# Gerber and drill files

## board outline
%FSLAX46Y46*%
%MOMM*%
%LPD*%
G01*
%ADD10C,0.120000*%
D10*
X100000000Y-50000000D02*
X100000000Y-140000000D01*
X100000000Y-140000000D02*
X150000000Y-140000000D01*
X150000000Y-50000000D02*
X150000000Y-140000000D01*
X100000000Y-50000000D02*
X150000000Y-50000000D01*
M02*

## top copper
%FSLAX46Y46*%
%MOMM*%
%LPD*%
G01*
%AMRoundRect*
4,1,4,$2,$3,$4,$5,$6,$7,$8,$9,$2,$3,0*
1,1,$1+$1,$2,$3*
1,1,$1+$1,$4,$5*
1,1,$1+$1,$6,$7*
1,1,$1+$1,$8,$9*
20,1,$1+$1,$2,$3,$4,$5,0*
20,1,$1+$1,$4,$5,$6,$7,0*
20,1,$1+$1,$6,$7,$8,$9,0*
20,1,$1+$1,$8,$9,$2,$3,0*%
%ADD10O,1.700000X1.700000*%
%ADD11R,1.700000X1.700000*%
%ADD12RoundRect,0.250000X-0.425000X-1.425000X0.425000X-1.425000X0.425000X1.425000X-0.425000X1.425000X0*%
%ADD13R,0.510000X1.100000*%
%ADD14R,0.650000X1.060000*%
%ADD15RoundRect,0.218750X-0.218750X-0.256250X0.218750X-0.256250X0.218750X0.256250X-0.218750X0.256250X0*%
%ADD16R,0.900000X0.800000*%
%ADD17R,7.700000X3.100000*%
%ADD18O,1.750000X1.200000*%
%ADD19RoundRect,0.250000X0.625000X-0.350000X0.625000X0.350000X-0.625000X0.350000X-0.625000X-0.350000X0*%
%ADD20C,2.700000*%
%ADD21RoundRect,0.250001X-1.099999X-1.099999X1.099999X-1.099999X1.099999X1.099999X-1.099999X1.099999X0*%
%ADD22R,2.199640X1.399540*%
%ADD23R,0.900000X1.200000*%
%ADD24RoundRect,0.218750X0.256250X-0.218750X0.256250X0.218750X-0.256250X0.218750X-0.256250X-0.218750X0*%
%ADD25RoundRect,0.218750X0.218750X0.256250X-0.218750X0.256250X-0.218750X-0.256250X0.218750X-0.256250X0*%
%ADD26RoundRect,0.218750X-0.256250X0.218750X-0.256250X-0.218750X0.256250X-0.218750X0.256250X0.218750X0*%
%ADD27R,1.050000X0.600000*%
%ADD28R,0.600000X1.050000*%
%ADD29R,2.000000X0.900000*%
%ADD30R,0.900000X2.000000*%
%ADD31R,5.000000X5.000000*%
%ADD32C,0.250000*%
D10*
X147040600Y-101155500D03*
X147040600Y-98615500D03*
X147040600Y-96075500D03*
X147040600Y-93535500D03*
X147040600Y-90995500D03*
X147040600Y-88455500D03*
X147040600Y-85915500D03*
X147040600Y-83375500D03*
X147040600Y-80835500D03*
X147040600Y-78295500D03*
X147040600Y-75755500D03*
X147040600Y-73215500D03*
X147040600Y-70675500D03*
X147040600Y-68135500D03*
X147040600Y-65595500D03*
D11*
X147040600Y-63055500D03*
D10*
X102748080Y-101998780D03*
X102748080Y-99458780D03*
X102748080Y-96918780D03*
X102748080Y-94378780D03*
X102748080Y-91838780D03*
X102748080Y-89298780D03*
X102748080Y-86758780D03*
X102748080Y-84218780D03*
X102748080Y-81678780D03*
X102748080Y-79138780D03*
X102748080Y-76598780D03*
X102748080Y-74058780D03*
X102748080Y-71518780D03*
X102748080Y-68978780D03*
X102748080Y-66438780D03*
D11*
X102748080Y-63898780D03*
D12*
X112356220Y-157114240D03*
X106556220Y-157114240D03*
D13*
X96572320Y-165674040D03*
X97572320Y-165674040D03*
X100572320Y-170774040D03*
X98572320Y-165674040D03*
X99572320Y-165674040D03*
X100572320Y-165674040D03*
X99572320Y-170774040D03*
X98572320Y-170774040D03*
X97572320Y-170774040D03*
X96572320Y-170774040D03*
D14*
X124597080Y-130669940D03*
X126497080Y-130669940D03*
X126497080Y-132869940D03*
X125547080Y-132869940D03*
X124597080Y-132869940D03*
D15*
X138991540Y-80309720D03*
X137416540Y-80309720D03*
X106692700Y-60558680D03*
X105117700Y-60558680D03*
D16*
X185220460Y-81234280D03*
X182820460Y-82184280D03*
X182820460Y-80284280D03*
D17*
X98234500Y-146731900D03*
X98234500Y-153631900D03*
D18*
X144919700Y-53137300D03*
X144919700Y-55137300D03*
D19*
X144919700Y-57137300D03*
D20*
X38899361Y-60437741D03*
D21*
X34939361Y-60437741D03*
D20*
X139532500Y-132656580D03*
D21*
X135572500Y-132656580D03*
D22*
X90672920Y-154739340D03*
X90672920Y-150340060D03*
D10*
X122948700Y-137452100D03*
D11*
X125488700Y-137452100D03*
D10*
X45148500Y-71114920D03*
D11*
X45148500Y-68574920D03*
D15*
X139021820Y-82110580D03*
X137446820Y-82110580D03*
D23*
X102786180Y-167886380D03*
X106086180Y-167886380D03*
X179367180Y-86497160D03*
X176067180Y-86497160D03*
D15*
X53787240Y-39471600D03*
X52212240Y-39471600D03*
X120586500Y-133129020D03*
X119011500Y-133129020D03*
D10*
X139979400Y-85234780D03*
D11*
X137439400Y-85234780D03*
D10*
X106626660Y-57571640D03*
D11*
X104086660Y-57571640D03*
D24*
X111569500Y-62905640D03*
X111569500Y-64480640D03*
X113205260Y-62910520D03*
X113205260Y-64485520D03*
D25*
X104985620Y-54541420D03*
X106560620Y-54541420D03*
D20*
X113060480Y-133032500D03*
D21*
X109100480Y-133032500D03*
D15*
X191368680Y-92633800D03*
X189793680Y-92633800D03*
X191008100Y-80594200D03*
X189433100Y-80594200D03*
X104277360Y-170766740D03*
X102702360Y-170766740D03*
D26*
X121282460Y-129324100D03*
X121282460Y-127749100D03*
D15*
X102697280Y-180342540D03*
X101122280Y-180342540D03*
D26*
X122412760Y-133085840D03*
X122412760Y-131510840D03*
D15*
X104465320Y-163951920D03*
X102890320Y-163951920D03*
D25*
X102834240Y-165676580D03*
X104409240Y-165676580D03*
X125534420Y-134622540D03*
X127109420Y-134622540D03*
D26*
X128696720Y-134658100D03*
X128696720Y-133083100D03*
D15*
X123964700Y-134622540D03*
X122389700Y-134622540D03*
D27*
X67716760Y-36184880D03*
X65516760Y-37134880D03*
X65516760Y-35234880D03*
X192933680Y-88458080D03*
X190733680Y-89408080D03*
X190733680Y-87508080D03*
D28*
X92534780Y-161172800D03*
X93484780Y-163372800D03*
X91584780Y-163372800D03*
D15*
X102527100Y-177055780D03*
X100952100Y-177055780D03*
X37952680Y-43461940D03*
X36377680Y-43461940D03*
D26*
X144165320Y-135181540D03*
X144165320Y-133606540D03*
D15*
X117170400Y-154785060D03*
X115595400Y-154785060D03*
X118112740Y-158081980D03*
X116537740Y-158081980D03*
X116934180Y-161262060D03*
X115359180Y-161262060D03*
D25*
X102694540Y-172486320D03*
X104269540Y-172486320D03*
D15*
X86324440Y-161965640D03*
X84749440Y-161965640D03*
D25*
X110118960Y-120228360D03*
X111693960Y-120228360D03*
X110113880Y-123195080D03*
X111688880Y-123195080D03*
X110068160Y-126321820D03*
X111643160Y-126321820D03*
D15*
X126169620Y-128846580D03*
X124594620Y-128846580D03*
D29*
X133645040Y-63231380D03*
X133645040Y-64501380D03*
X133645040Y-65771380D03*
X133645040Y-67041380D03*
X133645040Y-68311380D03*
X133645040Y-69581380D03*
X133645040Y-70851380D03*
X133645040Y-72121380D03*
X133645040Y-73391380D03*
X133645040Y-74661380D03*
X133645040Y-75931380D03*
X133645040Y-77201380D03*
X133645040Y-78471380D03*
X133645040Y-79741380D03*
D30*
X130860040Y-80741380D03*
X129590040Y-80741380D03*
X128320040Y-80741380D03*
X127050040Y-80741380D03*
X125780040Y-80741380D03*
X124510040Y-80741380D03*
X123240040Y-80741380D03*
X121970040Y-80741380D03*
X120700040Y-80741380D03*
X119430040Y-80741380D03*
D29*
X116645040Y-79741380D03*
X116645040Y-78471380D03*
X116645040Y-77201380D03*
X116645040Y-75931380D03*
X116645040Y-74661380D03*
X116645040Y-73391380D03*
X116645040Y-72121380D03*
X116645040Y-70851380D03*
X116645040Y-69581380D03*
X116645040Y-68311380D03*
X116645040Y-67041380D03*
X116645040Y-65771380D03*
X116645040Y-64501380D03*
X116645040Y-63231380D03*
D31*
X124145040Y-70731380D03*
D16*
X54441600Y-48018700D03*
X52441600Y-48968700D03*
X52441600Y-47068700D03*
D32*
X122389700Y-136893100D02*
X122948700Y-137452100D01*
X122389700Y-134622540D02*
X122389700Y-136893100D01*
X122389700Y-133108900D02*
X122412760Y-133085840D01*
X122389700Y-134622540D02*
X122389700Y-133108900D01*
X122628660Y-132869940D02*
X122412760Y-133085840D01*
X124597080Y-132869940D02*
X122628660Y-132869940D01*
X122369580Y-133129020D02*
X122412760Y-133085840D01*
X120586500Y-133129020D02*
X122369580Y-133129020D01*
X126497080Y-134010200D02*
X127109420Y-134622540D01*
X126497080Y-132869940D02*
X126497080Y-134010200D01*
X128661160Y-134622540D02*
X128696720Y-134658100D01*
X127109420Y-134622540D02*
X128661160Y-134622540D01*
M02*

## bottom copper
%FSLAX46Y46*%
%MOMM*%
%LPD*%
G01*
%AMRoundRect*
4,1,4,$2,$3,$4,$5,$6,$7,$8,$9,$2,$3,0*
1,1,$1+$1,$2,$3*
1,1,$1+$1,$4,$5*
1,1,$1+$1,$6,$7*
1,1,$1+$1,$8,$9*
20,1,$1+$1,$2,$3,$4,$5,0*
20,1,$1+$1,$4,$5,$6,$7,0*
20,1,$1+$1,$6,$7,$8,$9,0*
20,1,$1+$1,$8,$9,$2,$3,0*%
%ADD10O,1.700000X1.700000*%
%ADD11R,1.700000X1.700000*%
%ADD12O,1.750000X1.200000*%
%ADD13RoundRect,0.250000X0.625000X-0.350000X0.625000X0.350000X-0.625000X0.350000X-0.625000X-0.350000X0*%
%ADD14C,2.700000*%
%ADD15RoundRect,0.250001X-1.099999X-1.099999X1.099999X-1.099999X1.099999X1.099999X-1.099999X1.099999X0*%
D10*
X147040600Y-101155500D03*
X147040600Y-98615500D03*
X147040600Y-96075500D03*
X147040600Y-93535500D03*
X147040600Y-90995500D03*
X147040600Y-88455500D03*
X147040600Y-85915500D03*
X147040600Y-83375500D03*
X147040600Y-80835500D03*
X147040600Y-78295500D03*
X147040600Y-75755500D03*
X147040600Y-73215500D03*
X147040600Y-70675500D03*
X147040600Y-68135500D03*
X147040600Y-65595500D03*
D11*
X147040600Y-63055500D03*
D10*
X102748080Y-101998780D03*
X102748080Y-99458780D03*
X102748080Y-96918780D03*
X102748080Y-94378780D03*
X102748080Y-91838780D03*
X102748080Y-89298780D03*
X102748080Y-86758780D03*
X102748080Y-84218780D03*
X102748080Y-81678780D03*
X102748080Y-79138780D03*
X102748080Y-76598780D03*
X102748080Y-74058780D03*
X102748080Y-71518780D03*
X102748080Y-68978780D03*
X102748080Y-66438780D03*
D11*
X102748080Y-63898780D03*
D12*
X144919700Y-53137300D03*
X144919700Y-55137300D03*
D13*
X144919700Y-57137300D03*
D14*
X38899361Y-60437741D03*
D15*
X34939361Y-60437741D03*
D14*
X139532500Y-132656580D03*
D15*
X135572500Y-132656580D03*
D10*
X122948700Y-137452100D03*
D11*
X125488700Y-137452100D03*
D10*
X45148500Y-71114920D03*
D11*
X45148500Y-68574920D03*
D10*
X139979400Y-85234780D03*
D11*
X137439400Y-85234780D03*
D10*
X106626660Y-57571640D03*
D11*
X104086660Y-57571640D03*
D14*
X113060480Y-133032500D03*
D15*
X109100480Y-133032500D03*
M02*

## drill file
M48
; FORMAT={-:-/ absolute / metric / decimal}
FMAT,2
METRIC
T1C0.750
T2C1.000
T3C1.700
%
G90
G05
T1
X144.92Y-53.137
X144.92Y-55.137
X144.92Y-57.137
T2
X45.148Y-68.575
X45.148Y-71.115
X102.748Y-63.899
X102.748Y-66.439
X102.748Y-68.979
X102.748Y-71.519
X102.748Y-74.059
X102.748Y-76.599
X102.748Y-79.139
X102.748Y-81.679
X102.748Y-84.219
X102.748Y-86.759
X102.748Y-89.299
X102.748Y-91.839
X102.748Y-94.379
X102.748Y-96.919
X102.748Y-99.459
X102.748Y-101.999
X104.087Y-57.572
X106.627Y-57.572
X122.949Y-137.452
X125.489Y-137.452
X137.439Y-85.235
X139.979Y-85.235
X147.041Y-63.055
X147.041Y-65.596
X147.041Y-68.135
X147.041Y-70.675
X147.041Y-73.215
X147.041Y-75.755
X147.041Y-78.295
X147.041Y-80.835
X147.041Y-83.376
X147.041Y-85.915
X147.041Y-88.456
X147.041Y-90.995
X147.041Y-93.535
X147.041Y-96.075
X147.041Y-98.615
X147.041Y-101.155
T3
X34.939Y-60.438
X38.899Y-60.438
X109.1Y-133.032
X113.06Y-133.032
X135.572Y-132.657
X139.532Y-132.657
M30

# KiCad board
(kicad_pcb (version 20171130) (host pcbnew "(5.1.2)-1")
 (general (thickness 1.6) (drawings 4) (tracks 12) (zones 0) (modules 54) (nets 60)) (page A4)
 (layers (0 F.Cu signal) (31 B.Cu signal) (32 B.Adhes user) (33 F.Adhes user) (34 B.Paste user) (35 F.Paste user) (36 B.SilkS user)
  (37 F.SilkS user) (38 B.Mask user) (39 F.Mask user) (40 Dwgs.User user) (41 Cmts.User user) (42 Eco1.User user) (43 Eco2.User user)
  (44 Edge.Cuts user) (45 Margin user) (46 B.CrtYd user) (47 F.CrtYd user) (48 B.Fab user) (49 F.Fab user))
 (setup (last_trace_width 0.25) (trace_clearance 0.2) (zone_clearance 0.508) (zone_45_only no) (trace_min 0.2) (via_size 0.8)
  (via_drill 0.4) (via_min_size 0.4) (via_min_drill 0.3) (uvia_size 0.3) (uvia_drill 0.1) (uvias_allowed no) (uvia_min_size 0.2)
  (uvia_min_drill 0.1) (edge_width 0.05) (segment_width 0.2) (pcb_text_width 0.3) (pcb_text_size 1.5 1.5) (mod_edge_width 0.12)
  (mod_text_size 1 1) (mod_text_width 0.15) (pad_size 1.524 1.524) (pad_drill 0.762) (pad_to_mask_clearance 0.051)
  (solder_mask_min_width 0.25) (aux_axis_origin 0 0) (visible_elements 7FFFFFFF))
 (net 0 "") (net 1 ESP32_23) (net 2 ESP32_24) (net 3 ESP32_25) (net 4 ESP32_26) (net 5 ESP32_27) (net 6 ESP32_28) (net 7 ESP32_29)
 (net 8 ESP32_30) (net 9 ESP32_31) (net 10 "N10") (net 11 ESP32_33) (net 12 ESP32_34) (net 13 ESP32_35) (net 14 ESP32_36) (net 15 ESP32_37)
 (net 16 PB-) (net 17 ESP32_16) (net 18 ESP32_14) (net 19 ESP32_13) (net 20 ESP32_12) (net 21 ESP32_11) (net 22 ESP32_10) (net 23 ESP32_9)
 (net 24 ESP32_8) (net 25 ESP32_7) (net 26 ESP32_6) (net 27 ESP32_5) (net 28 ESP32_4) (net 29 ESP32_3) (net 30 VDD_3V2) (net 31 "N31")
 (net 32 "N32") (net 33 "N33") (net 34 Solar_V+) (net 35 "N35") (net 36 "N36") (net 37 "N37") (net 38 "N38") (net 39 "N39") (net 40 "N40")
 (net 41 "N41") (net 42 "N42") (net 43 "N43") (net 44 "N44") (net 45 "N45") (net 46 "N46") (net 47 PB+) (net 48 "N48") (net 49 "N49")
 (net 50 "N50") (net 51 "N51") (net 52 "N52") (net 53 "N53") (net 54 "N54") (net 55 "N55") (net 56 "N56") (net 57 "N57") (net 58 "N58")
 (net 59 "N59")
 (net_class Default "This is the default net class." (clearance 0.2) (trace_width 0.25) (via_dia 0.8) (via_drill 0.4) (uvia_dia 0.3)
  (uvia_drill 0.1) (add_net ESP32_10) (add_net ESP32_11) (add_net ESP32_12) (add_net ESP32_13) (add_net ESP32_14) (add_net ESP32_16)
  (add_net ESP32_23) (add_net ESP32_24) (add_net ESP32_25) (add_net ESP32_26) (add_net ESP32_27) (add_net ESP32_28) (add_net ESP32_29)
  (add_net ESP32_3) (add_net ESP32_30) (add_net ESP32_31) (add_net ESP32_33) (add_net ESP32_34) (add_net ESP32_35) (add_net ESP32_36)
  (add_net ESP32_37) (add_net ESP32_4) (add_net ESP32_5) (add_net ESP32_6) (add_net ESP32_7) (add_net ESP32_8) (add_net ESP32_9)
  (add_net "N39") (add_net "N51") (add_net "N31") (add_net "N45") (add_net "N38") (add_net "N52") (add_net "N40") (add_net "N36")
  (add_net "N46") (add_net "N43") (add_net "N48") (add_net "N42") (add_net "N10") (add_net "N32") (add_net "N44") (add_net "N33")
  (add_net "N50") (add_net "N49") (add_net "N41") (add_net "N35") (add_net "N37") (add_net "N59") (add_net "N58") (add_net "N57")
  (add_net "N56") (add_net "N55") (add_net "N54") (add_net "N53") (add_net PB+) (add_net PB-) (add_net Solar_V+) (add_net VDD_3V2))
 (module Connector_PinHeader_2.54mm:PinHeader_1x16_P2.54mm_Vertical (layer F.Cu) (at 147.0406 63.0555)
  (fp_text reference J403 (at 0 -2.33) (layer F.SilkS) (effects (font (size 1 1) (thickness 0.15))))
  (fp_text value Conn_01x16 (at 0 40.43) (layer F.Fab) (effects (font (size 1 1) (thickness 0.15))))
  (pad 16 thru_hole oval (at 0 38.1) (size 1.7 1.7) (drill 1) (layers *.Cu *.Mask) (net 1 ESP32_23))
  (pad 15 thru_hole oval (at 0 35.56) (size 1.7 1.7) (drill 1) (layers *.Cu *.Mask) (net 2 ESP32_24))
  (pad 14 thru_hole oval (at 0 33.02) (size 1.7 1.7) (drill 1) (layers *.Cu *.Mask) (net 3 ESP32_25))
  (pad 13 thru_hole oval (at 0 30.48) (size 1.7 1.7) (drill 1) (layers *.Cu *.Mask) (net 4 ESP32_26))
  (pad 12 thru_hole oval (at 0 27.94) (size 1.7 1.7) (drill 1) (layers *.Cu *.Mask) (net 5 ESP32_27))
  (pad 11 thru_hole oval (at 0 25.4) (size 1.7 1.7) (drill 1) (layers *.Cu *.Mask) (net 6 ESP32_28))
  (pad 10 thru_hole oval (at 0 22.86) (size 1.7 1.7) (drill 1) (layers *.Cu *.Mask) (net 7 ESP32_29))
  (pad 9 thru_hole oval (at 0 20.32) (size 1.7 1.7) (drill 1) (layers *.Cu *.Mask) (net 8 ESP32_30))
  (pad 8 thru_hole oval (at 0 17.78) (size 1.7 1.7) (drill 1) (layers *.Cu *.Mask) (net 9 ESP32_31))
  (pad 7 thru_hole oval (at 0 15.24) (size 1.7 1.7) (drill 1) (layers *.Cu *.Mask) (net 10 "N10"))
  (pad 6 thru_hole oval (at 0 12.7) (size 1.7 1.7) (drill 1) (layers *.Cu *.Mask) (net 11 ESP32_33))
  (pad 5 thru_hole oval (at 0 10.16) (size 1.7 1.7) (drill 1) (layers *.Cu *.Mask) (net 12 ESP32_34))
  (pad 4 thru_hole oval (at 0 7.62) (size 1.7 1.7) (drill 1) (layers *.Cu *.Mask) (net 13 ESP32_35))
  (pad 3 thru_hole oval (at 0 5.08) (size 1.7 1.7) (drill 1) (layers *.Cu *.Mask) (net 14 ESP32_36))
  (pad 2 thru_hole oval (at 0 2.54) (size 1.7 1.7) (drill 1) (layers *.Cu *.Mask) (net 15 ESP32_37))
  (pad 1 thru_hole rect (at 0 0) (size 1.7 1.7) (drill 1) (layers *.Cu *.Mask) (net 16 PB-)))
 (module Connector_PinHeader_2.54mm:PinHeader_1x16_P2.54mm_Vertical (layer F.Cu) (at 102.74808 63.89878)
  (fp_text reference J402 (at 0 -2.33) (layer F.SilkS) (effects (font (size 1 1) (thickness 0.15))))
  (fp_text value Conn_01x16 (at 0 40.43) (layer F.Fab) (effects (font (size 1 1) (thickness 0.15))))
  (pad 16 thru_hole oval (at 0 38.1) (size 1.7 1.7) (drill 1) (layers *.Cu *.Mask) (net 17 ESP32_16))
  (pad 15 thru_hole oval (at 0 35.56) (size 1.7 1.7) (drill 1) (layers *.Cu *.Mask) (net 16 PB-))
  (pad 14 thru_hole oval (at 0 33.02) (size 1.7 1.7) (drill 1) (layers *.Cu *.Mask) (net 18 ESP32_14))
  (pad 13 thru_hole oval (at 0 30.48) (size 1.7 1.7) (drill 1) (layers *.Cu *.Mask) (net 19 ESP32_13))
  (pad 12 thru_hole oval (at 0 27.94) (size 1.7 1.7) (drill 1) (layers *.Cu *.Mask) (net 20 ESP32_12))
  (pad 11 thru_hole oval (at 0 25.4) (size 1.7 1.7) (drill 1) (layers *.Cu *.Mask) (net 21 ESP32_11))
  (pad 10 thru_hole oval (at 0 22.86) (size 1.7 1.7) (drill 1) (layers *.Cu *.Mask) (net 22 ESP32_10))
  (pad 9 thru_hole oval (at 0 20.32) (size 1.7 1.7) (drill 1) (layers *.Cu *.Mask) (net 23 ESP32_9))
  (pad 8 thru_hole oval (at 0 17.78) (size 1.7 1.7) (drill 1) (layers *.Cu *.Mask) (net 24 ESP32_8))
  (pad 7 thru_hole oval (at 0 15.24) (size 1.7 1.7) (drill 1) (layers *.Cu *.Mask) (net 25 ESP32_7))
  (pad 6 thru_hole oval (at 0 12.7) (size 1.7 1.7) (drill 1) (layers *.Cu *.Mask) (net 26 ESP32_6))
  (pad 5 thru_hole oval (at 0 10.16) (size 1.7 1.7) (drill 1) (layers *.Cu *.Mask) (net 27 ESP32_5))
  (pad 4 thru_hole oval (at 0 7.62) (size 1.7 1.7) (drill 1) (layers *.Cu *.Mask) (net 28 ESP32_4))
  (pad 3 thru_hole oval (at 0 5.08) (size 1.7 1.7) (drill 1) (layers *.Cu *.Mask) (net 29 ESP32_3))
  (pad 2 thru_hole oval (at 0 2.54) (size 1.7 1.7) (drill 1) (layers *.Cu *.Mask) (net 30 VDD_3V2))
  (pad 1 thru_hole rect (at 0 0) (size 1.7 1.7) (drill 1) (layers *.Cu *.Mask) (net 16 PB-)))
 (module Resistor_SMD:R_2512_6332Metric (layer F.Cu) (at 109.45622 157.11424)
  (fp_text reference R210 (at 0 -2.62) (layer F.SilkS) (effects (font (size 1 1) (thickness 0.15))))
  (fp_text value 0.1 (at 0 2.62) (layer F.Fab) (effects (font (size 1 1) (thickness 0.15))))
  (pad 2 smd roundrect (at 2.9 0) (size 1.35 3.35) (layers F.Cu F.Paste F.Mask) (roundrect_rratio 0.185185) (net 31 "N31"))
  (pad 1 smd roundrect (at -2.9 0) (size 1.35 3.35) (layers F.Cu F.Paste F.Mask) (roundrect_rratio 0.185185) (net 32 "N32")))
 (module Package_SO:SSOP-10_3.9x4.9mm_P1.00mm (layer F.Cu) (at 98.57232 168.22404 90)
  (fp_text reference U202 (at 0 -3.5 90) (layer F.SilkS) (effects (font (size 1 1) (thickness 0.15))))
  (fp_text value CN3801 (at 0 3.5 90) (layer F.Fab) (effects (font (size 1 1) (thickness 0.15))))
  (pad 10 smd rect (at 2.55 -2 90) (size 1.1 0.51) (layers F.Cu F.Paste F.Mask) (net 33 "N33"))
  (pad 9 smd rect (at 2.55 -1 90) (size 1.1 0.51) (layers F.Cu F.Paste F.Mask) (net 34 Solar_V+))
  (pad 5 smd rect (at -2.55 2 90) (size 1.1 0.51) (layers F.Cu F.Paste F.Mask) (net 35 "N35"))
  (pad 8 smd rect (at 2.55 0 90) (size 1.1 0.51) (layers F.Cu F.Paste F.Mask) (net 32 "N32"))
  (pad 7 smd rect (at 2.55 1 90) (size 1.1 0.51) (layers F.Cu F.Paste F.Mask) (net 31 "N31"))
  (pad 6 smd rect (at 2.55 2 90) (size 1.1 0.51) (layers F.Cu F.Paste F.Mask) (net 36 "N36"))
  (pad 4 smd rect (at -2.55 1 90) (size 1.1 0.51) (layers F.Cu F.Paste F.Mask) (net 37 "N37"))
  (pad 3 smd rect (at -2.55 0 90) (size 1.1 0.51) (layers F.Cu F.Paste F.Mask) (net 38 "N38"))
  (pad 2 smd rect (at -2.55 -1 90) (size 1.1 0.51) (layers F.Cu F.Paste F.Mask) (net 16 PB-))
  (pad 1 smd rect (at -2.55 -2 90) (size 1.1 0.51) (layers F.Cu F.Paste F.Mask) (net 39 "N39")))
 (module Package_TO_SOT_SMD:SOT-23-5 (layer F.Cu) (at 125.54708 131.76994 90)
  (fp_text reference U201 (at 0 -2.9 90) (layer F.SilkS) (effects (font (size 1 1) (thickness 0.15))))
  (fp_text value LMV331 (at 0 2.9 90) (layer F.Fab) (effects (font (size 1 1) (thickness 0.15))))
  (pad 5 smd rect (at 1.1 -0.95 90) (size 1.06 0.65) (layers F.Cu F.Paste F.Mask) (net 34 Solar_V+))
  (pad 4 smd rect (at 1.1 0.95 90) (size 1.06 0.65) (layers F.Cu F.Paste F.Mask) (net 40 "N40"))
  (pad 3 smd rect (at -1.1 0.95 90) (size 1.06 0.65) (layers F.Cu F.Paste F.Mask) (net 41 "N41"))
  (pad 2 smd rect (at -1.1 0 90) (size 1.06 0.65) (layers F.Cu F.Paste F.Mask) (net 16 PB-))
  (pad 1 smd rect (at -1.1 -0.95 90) (size 1.06 0.65) (layers F.Cu F.Paste F.Mask) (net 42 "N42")))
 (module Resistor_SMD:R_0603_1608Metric (layer F.Cu) (at 138.20404 80.30972)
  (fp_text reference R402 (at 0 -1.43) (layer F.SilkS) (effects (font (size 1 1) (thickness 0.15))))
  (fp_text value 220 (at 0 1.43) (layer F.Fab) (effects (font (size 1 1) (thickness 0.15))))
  (pad 2 smd roundrect (at 0.7875 0) (size 0.875 0.95) (layers F.Cu F.Paste F.Mask) (roundrect_rratio 0.25) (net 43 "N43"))
  (pad 1 smd roundrect (at -0.7875 0) (size 0.875 0.95) (layers F.Cu F.Paste F.Mask) (roundrect_rratio 0.25) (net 30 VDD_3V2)))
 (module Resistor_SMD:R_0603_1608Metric (layer F.Cu) (at 105.9052 60.55868)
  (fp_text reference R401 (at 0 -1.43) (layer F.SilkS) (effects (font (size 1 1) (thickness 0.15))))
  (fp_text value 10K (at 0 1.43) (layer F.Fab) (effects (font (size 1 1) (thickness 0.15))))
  (pad 2 smd roundrect (at 0.7875 0) (size 0.875 0.95) (layers F.Cu F.Paste F.Mask) (roundrect_rratio 0.25) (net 29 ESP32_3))
  (pad 1 smd roundrect (at -0.7875 0) (size 0.875 0.95) (layers F.Cu F.Paste F.Mask) (roundrect_rratio 0.25) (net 30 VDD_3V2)))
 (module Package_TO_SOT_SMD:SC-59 (layer F.Cu) (at 184.02046 81.23428)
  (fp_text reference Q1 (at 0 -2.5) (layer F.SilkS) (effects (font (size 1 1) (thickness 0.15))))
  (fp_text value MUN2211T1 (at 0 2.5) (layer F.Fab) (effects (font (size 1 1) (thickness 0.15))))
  (pad 3 smd rect (at 1.2 0) (size 0.9 0.8) (layers F.Cu F.Paste F.Mask) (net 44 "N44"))
  (pad 2 smd rect (at -1.2 0.95) (size 0.9 0.8) (layers F.Cu F.Paste F.Mask) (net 16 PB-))
  (pad 1 smd rect (at -1.2 -0.95) (size 0.9 0.8) (layers F.Cu F.Paste F.Mask) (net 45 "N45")))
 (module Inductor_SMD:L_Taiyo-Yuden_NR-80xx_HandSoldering (layer F.Cu) (at 98.2345 150.1819 90)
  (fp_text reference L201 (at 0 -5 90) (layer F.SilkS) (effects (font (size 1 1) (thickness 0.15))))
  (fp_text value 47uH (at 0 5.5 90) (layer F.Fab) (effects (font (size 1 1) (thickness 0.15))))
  (pad 2 smd rect (at 3.45 0 90) (size 3.1 7.7) (layers F.Cu F.Paste F.Mask) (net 32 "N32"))
  (pad 1 smd rect (at -3.45 0 90) (size 3.1 7.7) (layers F.Cu F.Paste F.Mask) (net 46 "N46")))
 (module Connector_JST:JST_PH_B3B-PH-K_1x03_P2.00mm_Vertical (layer F.Cu) (at 144.9197 57.1373 90)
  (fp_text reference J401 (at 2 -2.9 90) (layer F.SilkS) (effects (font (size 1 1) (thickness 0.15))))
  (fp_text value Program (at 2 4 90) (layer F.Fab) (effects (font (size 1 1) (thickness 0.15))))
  (pad 3 thru_hole oval (at 4 0 90) (size 1.2 1.75) (drill 0.75) (layers *.Cu *.Mask) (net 13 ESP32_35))
  (pad 2 thru_hole oval (at 2 0 90) (size 1.2 1.75) (drill 0.75) (layers *.Cu *.Mask) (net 12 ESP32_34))
  (pad 1 thru_hole roundrect (at 0 0 90) (size 1.2 1.75) (drill 0.75) (layers *.Cu *.Mask) (roundrect_rratio 0.208333) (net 16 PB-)))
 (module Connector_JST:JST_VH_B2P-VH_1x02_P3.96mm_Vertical (layer F.Cu) (at 34.939361 60.437741)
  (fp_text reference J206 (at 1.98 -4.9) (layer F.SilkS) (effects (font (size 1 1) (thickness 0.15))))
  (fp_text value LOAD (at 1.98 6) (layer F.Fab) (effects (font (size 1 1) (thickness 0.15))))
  (pad 2 thru_hole circle (at 3.96 0) (size 2.7 2.7) (drill 1.7) (layers *.Cu *.Mask) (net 30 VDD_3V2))
  (pad 1 thru_hole roundrect (at 0 0) (size 2.7 2.7) (drill 1.7) (layers *.Cu *.Mask) (roundrect_rratio 0.09259299999999999) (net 16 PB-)))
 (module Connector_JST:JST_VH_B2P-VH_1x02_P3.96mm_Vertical (layer F.Cu) (at 135.5725 132.65658)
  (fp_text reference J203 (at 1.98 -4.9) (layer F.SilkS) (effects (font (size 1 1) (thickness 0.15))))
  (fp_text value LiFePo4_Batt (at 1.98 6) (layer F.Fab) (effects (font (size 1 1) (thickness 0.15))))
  (pad 2 thru_hole circle (at 3.96 0) (size 2.7 2.7) (drill 1.7) (layers *.Cu *.Mask) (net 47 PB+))
  (pad 1 thru_hole roundrect (at 0 0) (size 2.7 2.7) (drill 1.7) (layers *.Cu *.Mask) (roundrect_rratio 0.09259299999999999) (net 16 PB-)))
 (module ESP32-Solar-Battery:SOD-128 (layer F.Cu) (at 90.67292 152.5397 270)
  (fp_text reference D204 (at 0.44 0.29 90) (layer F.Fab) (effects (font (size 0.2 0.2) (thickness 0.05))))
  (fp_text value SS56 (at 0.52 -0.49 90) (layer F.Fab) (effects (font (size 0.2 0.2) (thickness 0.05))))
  (pad 1 smd rect (at 2.19964 0 270) (size 1.39954 2.19964) (layers F.Cu F.Paste F.Mask) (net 46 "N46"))
  (pad 2 smd rect (at -2.19964 0 270) (size 1.39954 2.19964) (layers F.Cu F.Paste F.Mask) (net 16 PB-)))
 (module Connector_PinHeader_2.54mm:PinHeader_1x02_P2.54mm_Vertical (layer F.Cu) (at 125.4887 137.4521 270)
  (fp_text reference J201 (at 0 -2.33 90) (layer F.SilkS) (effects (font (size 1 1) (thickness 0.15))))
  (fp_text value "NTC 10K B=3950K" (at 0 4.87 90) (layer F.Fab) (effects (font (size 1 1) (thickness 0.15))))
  (pad 2 thru_hole oval (at 0 2.54 270) (size 1.7 1.7) (drill 1) (layers *.Cu *.Mask) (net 42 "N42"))
  (pad 1 thru_hole rect (at 0 0 270) (size 1.7 1.7) (drill 1) (layers *.Cu *.Mask) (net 16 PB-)))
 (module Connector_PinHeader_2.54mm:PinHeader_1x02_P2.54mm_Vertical (layer F.Cu) (at 45.1485 68.57492)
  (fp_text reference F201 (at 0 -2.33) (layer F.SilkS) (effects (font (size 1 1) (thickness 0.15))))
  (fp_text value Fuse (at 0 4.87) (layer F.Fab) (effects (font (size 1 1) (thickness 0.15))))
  (pad 2 thru_hole oval (at 0 2.54) (size 1.7 1.7) (drill 1) (layers *.Cu *.Mask) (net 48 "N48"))
  (pad 1 thru_hole rect (at 0 0) (size 1.7 1.7) (drill 1) (layers *.Cu *.Mask) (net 30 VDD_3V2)))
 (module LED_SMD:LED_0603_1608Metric (layer F.Cu) (at 138.23432 82.11058)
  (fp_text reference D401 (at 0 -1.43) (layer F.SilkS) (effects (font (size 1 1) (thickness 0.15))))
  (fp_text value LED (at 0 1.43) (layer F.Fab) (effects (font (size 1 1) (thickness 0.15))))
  (pad 2 smd roundrect (at 0.7875 0) (size 0.875 0.95) (layers F.Cu F.Paste F.Mask) (roundrect_rratio 0.25) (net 43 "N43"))
  (pad 1 smd roundrect (at -0.7875 0) (size 0.875 0.95) (layers F.Cu F.Paste F.Mask) (roundrect_rratio 0.25) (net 3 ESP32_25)))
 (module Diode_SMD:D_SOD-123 (layer F.Cu) (at 104.43618 167.88638 180)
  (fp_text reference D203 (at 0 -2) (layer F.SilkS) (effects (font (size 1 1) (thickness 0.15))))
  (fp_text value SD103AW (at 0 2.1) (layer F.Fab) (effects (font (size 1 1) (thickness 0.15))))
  (pad 2 smd rect (at 1.65 0 180) (size 0.9 1.2) (layers F.Cu F.Paste F.Mask) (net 36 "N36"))
  (pad 1 smd rect (at -1.65 0 180) (size 0.9 1.2) (layers F.Cu F.Paste F.Mask) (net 40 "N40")))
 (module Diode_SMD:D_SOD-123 (layer F.Cu) (at 177.71718 86.49716)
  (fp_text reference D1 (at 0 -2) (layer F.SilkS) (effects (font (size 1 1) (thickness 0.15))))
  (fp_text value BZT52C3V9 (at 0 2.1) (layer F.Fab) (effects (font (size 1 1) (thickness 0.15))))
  (pad 2 smd rect (at 1.65 0) (size 0.9 1.2) (layers F.Cu F.Paste F.Mask) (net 45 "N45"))
  (pad 1 smd rect (at -1.65 0) (size 0.9 1.2) (layers F.Cu F.Paste F.Mask) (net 34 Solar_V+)))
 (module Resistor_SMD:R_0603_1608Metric (layer F.Cu) (at 52.99974 39.4716)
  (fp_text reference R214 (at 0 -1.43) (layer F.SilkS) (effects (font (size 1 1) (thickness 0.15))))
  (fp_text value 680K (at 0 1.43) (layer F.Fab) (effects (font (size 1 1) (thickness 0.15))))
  (pad 2 smd roundrect (at 0.7875 0) (size 0.875 0.95) (layers F.Cu F.Paste F.Mask) (roundrect_rratio 0.25) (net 47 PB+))
  (pad 1 smd roundrect (at -0.7875 0) (size 0.875 0.95) (layers F.Cu F.Paste F.Mask) (roundrect_rratio 0.25) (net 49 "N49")))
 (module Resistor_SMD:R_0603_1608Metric (layer F.Cu) (at 119.799 133.12902)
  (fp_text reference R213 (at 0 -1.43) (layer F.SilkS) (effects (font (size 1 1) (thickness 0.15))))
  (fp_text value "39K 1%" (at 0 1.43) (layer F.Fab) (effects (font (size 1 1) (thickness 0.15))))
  (pad 2 smd roundrect (at 0.7875 0) (size 0.875 0.95) (layers F.Cu F.Paste F.Mask) (roundrect_rratio 0.25) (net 42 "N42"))
  (pad 1 smd roundrect (at -0.7875 0) (size 0.875 0.95) (layers F.Cu F.Paste F.Mask) (roundrect_rratio 0.25) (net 34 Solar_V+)))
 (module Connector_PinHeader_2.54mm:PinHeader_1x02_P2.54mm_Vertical (layer F.Cu) (at 137.4394 85.23478 90)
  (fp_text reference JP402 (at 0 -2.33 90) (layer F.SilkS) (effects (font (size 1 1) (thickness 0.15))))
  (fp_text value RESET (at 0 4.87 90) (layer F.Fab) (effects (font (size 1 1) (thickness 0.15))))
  (pad 2 thru_hole oval (at 0 2.54 90) (size 1.7 1.7) (drill 1) (layers *.Cu *.Mask) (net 16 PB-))
  (pad 1 thru_hole rect (at 0 0 90) (size 1.7 1.7) (drill 1) (layers *.Cu *.Mask) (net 3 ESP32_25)))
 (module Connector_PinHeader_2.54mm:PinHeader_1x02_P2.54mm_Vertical (layer F.Cu) (at 104.08666 57.57164 90)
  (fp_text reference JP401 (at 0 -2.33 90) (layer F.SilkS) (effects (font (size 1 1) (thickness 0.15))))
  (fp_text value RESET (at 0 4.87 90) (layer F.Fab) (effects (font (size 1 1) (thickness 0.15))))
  (pad 2 thru_hole oval (at 0 2.54 90) (size 1.7 1.7) (drill 1) (layers *.Cu *.Mask) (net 29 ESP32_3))
  (pad 1 thru_hole rect (at 0 0 90) (size 1.7 1.7) (drill 1) (layers *.Cu *.Mask) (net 16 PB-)))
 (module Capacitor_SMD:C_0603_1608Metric (layer F.Cu) (at 111.5695 63.69314 90)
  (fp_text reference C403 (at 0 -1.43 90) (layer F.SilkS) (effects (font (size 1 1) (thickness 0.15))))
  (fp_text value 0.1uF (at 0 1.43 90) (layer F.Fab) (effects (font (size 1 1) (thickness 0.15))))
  (pad 2 smd roundrect (at 0.7875 0 90) (size 0.875 0.95) (layers F.Cu F.Paste F.Mask) (roundrect_rratio 0.25) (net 16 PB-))
  (pad 1 smd roundrect (at -0.7875 0 90) (size 0.875 0.95) (layers F.Cu F.Paste F.Mask) (roundrect_rratio 0.25) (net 30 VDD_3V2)))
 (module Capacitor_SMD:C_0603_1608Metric (layer F.Cu) (at 113.20526 63.69802 90)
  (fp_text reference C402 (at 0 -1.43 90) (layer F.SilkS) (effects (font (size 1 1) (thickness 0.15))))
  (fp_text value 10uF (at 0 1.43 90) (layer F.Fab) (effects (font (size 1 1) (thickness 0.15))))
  (pad 2 smd roundrect (at 0.7875 0 90) (size 0.875 0.95) (layers F.Cu F.Paste F.Mask) (roundrect_rratio 0.25) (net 16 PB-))
  (pad 1 smd roundrect (at -0.7875 0 90) (size 0.875 0.95) (layers F.Cu F.Paste F.Mask) (roundrect_rratio 0.25) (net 30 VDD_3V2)))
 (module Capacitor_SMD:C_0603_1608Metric (layer F.Cu) (at 105.77312 54.54142 180)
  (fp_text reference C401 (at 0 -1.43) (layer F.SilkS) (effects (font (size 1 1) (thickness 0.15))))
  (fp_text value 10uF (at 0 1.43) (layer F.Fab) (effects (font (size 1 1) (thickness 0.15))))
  (pad 2 smd roundrect (at 0.7875 0 180) (size 0.875 0.95) (layers F.Cu F.Paste F.Mask) (roundrect_rratio 0.25) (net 16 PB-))
  (pad 1 smd roundrect (at -0.7875 0 180) (size 0.875 0.95) (layers F.Cu F.Paste F.Mask) (roundrect_rratio 0.25) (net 29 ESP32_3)))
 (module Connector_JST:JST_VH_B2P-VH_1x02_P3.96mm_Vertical (layer F.Cu) (at 109.10048 133.0325)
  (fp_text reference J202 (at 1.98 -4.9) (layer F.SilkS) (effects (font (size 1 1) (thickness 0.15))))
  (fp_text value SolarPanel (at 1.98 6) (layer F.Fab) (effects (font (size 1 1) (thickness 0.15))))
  (pad 2 thru_hole circle (at 3.96 0) (size 2.7 2.7) (drill 1.7) (layers *.Cu *.Mask) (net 34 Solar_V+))
  (pad 1 thru_hole roundrect (at 0 0) (size 2.7 2.7) (drill 1.7) (layers *.Cu *.Mask) (roundrect_rratio 0.09259299999999999) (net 16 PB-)))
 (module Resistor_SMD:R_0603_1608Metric (layer F.Cu) (at 190.58118 92.6338)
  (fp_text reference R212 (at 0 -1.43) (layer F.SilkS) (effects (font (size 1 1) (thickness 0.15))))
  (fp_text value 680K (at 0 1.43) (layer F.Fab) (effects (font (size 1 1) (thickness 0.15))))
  (pad 2 smd roundrect (at 0.7875 0) (size 0.875 0.95) (layers F.Cu F.Paste F.Mask) (roundrect_rratio 0.25) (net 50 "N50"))
  (pad 1 smd roundrect (at -0.7875 0) (size 0.875 0.95) (layers F.Cu F.Paste F.Mask) (roundrect_rratio 0.25) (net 47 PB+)))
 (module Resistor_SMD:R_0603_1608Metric (layer F.Cu) (at 190.2206 80.5942)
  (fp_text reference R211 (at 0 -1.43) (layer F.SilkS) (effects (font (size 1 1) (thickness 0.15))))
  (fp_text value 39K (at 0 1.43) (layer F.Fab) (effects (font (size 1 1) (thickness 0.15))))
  (pad 2 smd roundrect (at 0.7875 0) (size 0.875 0.95) (layers F.Cu F.Paste F.Mask) (roundrect_rratio 0.25) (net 44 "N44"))
  (pad 1 smd roundrect (at -0.7875 0) (size 0.875 0.95) (layers F.Cu F.Paste F.Mask) (roundrect_rratio 0.25) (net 50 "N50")))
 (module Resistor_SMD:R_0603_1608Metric (layer F.Cu) (at 103.48986 170.76674)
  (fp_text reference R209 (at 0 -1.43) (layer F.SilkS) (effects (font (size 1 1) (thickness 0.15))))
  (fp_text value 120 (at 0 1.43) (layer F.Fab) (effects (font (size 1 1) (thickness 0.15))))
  (pad 2 smd roundrect (at 0.7875 0) (size 0.875 0.95) (layers F.Cu F.Paste F.Mask) (roundrect_rratio 0.25) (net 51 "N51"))
  (pad 1 smd roundrect (at -0.7875 0) (size 0.875 0.95) (layers F.Cu F.Paste F.Mask) (roundrect_rratio 0.25) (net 35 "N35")))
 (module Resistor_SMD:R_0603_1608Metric (layer F.Cu) (at 121.28246 128.5366 270)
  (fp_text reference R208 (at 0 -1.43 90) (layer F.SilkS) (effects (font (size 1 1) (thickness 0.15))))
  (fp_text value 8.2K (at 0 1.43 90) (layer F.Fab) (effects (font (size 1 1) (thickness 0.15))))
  (pad 2 smd roundrect (at 0.7875 0 270) (size 0.875 0.95) (layers F.Cu F.Paste F.Mask) (roundrect_rratio 0.25) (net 40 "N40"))
  (pad 1 smd roundrect (at -0.7875 0 270) (size 0.875 0.95) (layers F.Cu F.Paste F.Mask) (roundrect_rratio 0.25) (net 34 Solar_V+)))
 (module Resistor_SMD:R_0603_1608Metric (layer F.Cu) (at 101.90978 180.34254)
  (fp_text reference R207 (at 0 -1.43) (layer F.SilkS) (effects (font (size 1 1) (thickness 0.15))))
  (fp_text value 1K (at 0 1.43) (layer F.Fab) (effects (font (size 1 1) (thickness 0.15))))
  (pad 2 smd roundrect (at 0.7875 0) (size 0.875 0.95) (layers F.Cu F.Paste F.Mask) (roundrect_rratio 0.25) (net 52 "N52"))
  (pad 1 smd roundrect (at -0.7875 0) (size 0.875 0.95) (layers F.Cu F.Paste F.Mask) (roundrect_rratio 0.25) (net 34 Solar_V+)))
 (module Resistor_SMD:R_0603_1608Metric (layer F.Cu) (at 122.41276 132.29834 270)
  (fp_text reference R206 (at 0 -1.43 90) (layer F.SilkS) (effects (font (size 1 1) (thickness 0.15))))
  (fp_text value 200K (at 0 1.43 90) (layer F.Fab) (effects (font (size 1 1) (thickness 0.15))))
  (pad 2 smd roundrect (at 0.7875 0 270) (size 0.875 0.95) (layers F.Cu F.Paste F.Mask) (roundrect_rratio 0.25) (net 42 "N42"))
  (pad 1 smd roundrect (at -0.7875 0 270) (size 0.875 0.95) (layers F.Cu F.Paste F.Mask) (roundrect_rratio 0.25) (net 40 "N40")))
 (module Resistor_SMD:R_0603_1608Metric (layer F.Cu) (at 103.67782 163.95192)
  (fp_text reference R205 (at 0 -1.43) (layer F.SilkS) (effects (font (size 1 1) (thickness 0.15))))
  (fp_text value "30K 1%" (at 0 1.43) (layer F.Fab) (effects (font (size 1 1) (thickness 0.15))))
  (pad 2 smd roundrect (at 0.7875 0) (size 0.875 0.95) (layers F.Cu F.Paste F.Mask) (roundrect_rratio 0.25) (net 16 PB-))
  (pad 1 smd roundrect (at -0.7875 0) (size 0.875 0.95) (layers F.Cu F.Paste F.Mask) (roundrect_rratio 0.25) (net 36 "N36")))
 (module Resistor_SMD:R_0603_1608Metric (layer F.Cu) (at 103.62174 165.67658 180)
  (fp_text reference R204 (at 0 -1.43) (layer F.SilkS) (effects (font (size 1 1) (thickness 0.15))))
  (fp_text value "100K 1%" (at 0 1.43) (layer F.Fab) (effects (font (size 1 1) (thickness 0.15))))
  (pad 2 smd roundrect (at 0.7875 0 180) (size 0.875 0.95) (layers F.Cu F.Paste F.Mask) (roundrect_rratio 0.25) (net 36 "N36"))
  (pad 1 smd roundrect (at -0.7875 0 180) (size 0.875 0.95) (layers F.Cu F.Paste F.Mask) (roundrect_rratio 0.25) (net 34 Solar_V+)))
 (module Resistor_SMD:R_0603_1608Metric (layer F.Cu) (at 126.32192 134.62254 180)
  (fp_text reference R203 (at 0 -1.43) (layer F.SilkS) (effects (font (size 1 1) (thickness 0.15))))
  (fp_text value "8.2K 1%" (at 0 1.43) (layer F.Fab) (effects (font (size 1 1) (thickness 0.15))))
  (pad 2 smd roundrect (at 0.7875 0 180) (size 0.875 0.95) (layers F.Cu F.Paste F.Mask) (roundrect_rratio 0.25) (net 16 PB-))
  (pad 1 smd roundrect (at -0.7875 0 180) (size 0.875 0.95) (layers F.Cu F.Paste F.Mask) (roundrect_rratio 0.25) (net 41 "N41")))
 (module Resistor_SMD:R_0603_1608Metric (layer F.Cu) (at 128.69672 133.8706 270)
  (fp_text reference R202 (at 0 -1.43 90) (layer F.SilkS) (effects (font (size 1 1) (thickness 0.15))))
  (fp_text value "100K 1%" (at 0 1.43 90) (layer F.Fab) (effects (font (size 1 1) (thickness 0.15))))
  (pad 2 smd roundrect (at 0.7875 0 270) (size 0.875 0.95) (layers F.Cu F.Paste F.Mask) (roundrect_rratio 0.25) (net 41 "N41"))
  (pad 1 smd roundrect (at -0.7875 0 270) (size 0.875 0.95) (layers F.Cu F.Paste F.Mask) (roundrect_rratio 0.25) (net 34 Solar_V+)))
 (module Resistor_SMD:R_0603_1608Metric (layer F.Cu) (at 123.1772 134.62254)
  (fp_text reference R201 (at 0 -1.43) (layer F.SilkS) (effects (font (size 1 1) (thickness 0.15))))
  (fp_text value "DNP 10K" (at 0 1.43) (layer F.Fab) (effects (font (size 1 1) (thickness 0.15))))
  (pad 2 smd roundrect (at 0.7875 0) (size 0.875 0.95) (layers F.Cu F.Paste F.Mask) (roundrect_rratio 0.25) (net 16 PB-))
  (pad 1 smd roundrect (at -0.7875 0) (size 0.875 0.95) (layers F.Cu F.Paste F.Mask) (roundrect_rratio 0.25) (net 42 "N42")))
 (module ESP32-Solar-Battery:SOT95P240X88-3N (layer F.Cu) (at 66.61676 36.18488)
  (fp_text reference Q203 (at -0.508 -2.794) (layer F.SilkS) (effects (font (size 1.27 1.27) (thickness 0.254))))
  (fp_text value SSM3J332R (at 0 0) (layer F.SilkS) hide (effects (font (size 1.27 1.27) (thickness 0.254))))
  (pad 3 smd rect (at 1.1 0 90) (size 0.6 1.05) (layers F.Cu F.Paste F.Mask) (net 48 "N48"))
  (pad 2 smd rect (at -1.1 0.95 90) (size 0.6 1.05) (layers F.Cu F.Paste F.Mask) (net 47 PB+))
  (pad 1 smd rect (at -1.1 -0.95 90) (size 0.6 1.05) (layers F.Cu F.Paste F.Mask) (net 49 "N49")))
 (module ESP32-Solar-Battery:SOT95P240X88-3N (layer F.Cu) (at 191.83368 88.45808)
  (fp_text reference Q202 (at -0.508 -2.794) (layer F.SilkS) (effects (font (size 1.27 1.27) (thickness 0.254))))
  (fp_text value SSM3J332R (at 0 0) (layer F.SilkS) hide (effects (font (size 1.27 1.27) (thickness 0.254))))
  (pad 3 smd rect (at 1.1 0 90) (size 0.6 1.05) (layers F.Cu F.Paste F.Mask) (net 31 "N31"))
  (pad 2 smd rect (at -1.1 0.95 90) (size 0.6 1.05) (layers F.Cu F.Paste F.Mask) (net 47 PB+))
  (pad 1 smd rect (at -1.1 -0.95 90) (size 0.6 1.05) (layers F.Cu F.Paste F.Mask) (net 50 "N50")))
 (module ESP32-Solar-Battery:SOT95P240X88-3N (layer F.Cu) (at 92.53478 162.2728 90)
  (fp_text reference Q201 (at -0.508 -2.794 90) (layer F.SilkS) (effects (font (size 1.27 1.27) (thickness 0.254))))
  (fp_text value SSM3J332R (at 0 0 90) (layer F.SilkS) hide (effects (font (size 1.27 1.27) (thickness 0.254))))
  (pad 3 smd rect (at 1.1 0 180) (size 0.6 1.05) (layers F.Cu F.Paste F.Mask) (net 46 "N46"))
  (pad 2 smd rect (at -1.1 0.95 180) (size 0.6 1.05) (layers F.Cu F.Paste F.Mask) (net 34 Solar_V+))
  (pad 1 smd rect (at -1.1 -0.95 180) (size 0.6 1.05) (layers F.Cu F.Paste F.Mask) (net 33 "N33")))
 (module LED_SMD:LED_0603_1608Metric (layer F.Cu) (at 101.7396 177.05578)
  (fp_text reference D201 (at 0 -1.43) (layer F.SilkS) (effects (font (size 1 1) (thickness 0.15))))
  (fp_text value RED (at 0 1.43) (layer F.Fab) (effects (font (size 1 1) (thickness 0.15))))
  (pad 2 smd roundrect (at 0.7875 0) (size 0.875 0.95) (layers F.Cu F.Paste F.Mask) (roundrect_rratio 0.25) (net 52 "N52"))
  (pad 1 smd roundrect (at -0.7875 0) (size 0.875 0.95) (layers F.Cu F.Paste F.Mask) (roundrect_rratio 0.25) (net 38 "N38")))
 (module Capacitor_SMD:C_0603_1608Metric (layer F.Cu) (at 37.16518 43.46194)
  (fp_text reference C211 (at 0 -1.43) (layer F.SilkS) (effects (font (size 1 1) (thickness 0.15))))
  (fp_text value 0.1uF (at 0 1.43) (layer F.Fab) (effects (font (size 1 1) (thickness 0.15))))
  (pad 2 smd roundrect (at 0.7875 0) (size 0.875 0.95) (layers F.Cu F.Paste F.Mask) (roundrect_rratio 0.25) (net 16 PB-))
  (pad 1 smd roundrect (at -0.7875 0) (size 0.875 0.95) (layers F.Cu F.Paste F.Mask) (roundrect_rratio 0.25) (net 30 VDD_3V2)))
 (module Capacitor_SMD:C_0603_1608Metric (layer F.Cu) (at 144.16532 134.39404 270)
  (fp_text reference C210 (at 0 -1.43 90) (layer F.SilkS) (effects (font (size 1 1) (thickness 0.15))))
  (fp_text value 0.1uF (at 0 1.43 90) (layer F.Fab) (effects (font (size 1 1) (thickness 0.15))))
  (pad 2 smd roundrect (at 0.7875 0 270) (size 0.875 0.95) (layers F.Cu F.Paste F.Mask) (roundrect_rratio 0.25) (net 16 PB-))
  (pad 1 smd roundrect (at -0.7875 0 270) (size 0.875 0.95) (layers F.Cu F.Paste F.Mask) (roundrect_rratio 0.25) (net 47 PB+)))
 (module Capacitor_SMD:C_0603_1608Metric (layer F.Cu) (at 116.3829 154.78506)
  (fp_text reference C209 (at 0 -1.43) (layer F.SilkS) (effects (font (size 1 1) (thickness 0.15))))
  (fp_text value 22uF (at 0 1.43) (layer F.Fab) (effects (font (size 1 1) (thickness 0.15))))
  (pad 2 smd roundrect (at 0.7875 0) (size 0.875 0.95) (layers F.Cu F.Paste F.Mask) (roundrect_rratio 0.25) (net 16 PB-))
  (pad 1 smd roundrect (at -0.7875 0) (size 0.875 0.95) (layers F.Cu F.Paste F.Mask) (roundrect_rratio 0.25) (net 31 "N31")))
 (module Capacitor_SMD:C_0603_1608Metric (layer F.Cu) (at 117.32524 158.08198)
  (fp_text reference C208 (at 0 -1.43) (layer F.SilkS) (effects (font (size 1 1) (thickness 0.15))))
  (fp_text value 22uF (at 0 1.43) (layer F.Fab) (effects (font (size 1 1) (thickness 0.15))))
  (pad 2 smd roundrect (at 0.7875 0) (size 0.875 0.95) (layers F.Cu F.Paste F.Mask) (roundrect_rratio 0.25) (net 16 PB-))
  (pad 1 smd roundrect (at -0.7875 0) (size 0.875 0.95) (layers F.Cu F.Paste F.Mask) (roundrect_rratio 0.25) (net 31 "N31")))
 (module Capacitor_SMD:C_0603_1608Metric (layer F.Cu) (at 116.14668 161.26206)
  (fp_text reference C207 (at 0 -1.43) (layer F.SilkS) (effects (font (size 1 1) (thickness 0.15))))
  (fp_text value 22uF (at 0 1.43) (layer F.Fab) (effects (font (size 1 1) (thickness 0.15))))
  (pad 2 smd roundrect (at 0.7875 0) (size 0.875 0.95) (layers F.Cu F.Paste F.Mask) (roundrect_rratio 0.25) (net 16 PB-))
  (pad 1 smd roundrect (at -0.7875 0) (size 0.875 0.95) (layers F.Cu F.Paste F.Mask) (roundrect_rratio 0.25) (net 31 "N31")))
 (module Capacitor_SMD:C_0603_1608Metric (layer F.Cu) (at 103.48204 172.48632 180)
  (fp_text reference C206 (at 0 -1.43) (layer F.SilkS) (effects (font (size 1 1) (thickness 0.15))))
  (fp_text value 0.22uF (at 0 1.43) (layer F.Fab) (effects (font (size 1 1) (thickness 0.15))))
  (pad 2 smd roundrect (at 0.7875 0 180) (size 0.875 0.95) (layers F.Cu F.Paste F.Mask) (roundrect_rratio 0.25) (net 16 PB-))
  (pad 1 smd roundrect (at -0.7875 0 180) (size 0.875 0.95) (layers F.Cu F.Paste F.Mask) (roundrect_rratio 0.25) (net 51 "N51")))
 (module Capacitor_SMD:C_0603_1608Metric (layer F.Cu) (at 85.53694 161.96564)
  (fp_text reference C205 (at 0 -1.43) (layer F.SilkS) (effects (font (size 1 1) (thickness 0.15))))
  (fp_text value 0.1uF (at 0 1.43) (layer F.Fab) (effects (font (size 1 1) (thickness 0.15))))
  (pad 2 smd roundrect (at 0.7875 0) (size 0.875 0.95) (layers F.Cu F.Paste F.Mask) (roundrect_rratio 0.25) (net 39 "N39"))
  (pad 1 smd roundrect (at -0.7875 0) (size 0.875 0.95) (layers F.Cu F.Paste F.Mask) (roundrect_rratio 0.25) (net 34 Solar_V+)))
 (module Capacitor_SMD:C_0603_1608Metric (layer F.Cu) (at 110.90646 120.22836 180)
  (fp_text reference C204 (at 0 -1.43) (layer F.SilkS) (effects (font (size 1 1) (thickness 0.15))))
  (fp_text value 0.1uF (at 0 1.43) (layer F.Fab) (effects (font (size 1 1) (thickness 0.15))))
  (pad 2 smd roundrect (at 0.7875 0 180) (size 0.875 0.95) (layers F.Cu F.Paste F.Mask) (roundrect_rratio 0.25) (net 16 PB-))
  (pad 1 smd roundrect (at -0.7875 0 180) (size 0.875 0.95) (layers F.Cu F.Paste F.Mask) (roundrect_rratio 0.25) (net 34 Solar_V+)))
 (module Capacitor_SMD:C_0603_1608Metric (layer F.Cu) (at 110.90138 123.19508 180)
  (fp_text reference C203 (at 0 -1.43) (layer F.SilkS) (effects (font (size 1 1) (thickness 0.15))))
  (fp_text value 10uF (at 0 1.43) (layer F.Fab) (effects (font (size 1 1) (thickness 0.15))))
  (pad 2 smd roundrect (at 0.7875 0 180) (size 0.875 0.95) (layers F.Cu F.Paste F.Mask) (roundrect_rratio 0.25) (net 16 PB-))
  (pad 1 smd roundrect (at -0.7875 0 180) (size 0.875 0.95) (layers F.Cu F.Paste F.Mask) (roundrect_rratio 0.25) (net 34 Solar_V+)))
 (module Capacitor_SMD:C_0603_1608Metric (layer F.Cu) (at 110.85566 126.32182 180)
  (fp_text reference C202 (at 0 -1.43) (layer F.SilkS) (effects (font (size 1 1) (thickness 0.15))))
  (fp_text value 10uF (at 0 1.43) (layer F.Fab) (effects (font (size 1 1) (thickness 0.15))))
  (pad 2 smd roundrect (at 0.7875 0 180) (size 0.875 0.95) (layers F.Cu F.Paste F.Mask) (roundrect_rratio 0.25) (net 16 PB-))
  (pad 1 smd roundrect (at -0.7875 0 180) (size 0.875 0.95) (layers F.Cu F.Paste F.Mask) (roundrect_rratio 0.25) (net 34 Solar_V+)))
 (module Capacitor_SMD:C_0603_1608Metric (layer F.Cu) (at 125.38212 128.84658)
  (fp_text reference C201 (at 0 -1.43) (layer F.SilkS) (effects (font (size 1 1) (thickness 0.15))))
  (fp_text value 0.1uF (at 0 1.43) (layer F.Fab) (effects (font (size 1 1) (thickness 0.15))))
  (pad 2 smd roundrect (at 0.7875 0) (size 0.875 0.95) (layers F.Cu F.Paste F.Mask) (roundrect_rratio 0.25) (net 16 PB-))
  (pad 1 smd roundrect (at -0.7875 0) (size 0.875 0.95) (layers F.Cu F.Paste F.Mask) (roundrect_rratio 0.25) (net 34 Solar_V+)))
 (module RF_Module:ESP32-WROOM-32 (layer F.Cu) (at 125.14504 71.48638)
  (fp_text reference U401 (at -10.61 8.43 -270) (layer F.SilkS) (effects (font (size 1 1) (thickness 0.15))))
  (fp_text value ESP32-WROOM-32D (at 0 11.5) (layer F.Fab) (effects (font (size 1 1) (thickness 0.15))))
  (pad 38 smd rect (at 8.5 -8.255) (size 2 0.9) (layers F.Cu F.Paste F.Mask) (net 16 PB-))
  (pad 37 smd rect (at 8.5 -6.985) (size 2 0.9) (layers F.Cu F.Paste F.Mask) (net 15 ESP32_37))
  (pad 36 smd rect (at 8.5 -5.715) (size 2 0.9) (layers F.Cu F.Paste F.Mask) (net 14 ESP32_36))
  (pad 35 smd rect (at 8.5 -4.445) (size 2 0.9) (layers F.Cu F.Paste F.Mask) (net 13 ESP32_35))
  (pad 34 smd rect (at 8.5 -3.175) (size 2 0.9) (layers F.Cu F.Paste F.Mask) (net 12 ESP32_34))
  (pad 33 smd rect (at 8.5 -1.905) (size 2 0.9) (layers F.Cu F.Paste F.Mask) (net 11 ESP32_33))
  (pad 32 smd rect (at 8.5 -0.635) (size 2 0.9) (layers F.Cu F.Paste F.Mask) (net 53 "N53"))
  (pad 31 smd rect (at 8.5 0.635) (size 2 0.9) (layers F.Cu F.Paste F.Mask) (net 9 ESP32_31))
  (pad 30 smd rect (at 8.5 1.905) (size 2 0.9) (layers F.Cu F.Paste F.Mask) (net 8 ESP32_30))
  (pad 29 smd rect (at 8.5 3.175) (size 2 0.9) (layers F.Cu F.Paste F.Mask) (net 7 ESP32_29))
  (pad 28 smd rect (at 8.5 4.445) (size 2 0.9) (layers F.Cu F.Paste F.Mask) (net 6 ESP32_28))
  (pad 27 smd rect (at 8.5 5.715) (size 2 0.9) (layers F.Cu F.Paste F.Mask) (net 5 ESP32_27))
  (pad 26 smd rect (at 8.5 6.985) (size 2 0.9) (layers F.Cu F.Paste F.Mask) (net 4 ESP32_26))
  (pad 25 smd rect (at 8.5 8.255) (size 2 0.9) (layers F.Cu F.Paste F.Mask) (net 3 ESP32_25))
  (pad 24 smd rect (at 5.715 9.255 90) (size 2 0.9) (layers F.Cu F.Paste F.Mask) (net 2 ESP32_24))
  (pad 23 smd rect (at 4.445 9.255 90) (size 2 0.9) (layers F.Cu F.Paste F.Mask) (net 1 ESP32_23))
  (pad 22 smd rect (at 3.175 9.255 90) (size 2 0.9) (layers F.Cu F.Paste F.Mask) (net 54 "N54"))
  (pad 21 smd rect (at 1.905 9.255 90) (size 2 0.9) (layers F.Cu F.Paste F.Mask) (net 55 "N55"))
  (pad 20 smd rect (at 0.635 9.255 90) (size 2 0.9) (layers F.Cu F.Paste F.Mask) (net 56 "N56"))
  (pad 19 smd rect (at -0.635 9.255 90) (size 2 0.9) (layers F.Cu F.Paste F.Mask) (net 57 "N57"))
  (pad 18 smd rect (at -1.905 9.255 90) (size 2 0.9) (layers F.Cu F.Paste F.Mask) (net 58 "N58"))
  (pad 17 smd rect (at -3.175 9.255 90) (size 2 0.9) (layers F.Cu F.Paste F.Mask) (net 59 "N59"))
  (pad 16 smd rect (at -4.445 9.255 90) (size 2 0.9) (layers F.Cu F.Paste F.Mask) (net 17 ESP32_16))
  (pad 15 smd rect (at -5.715 9.255 90) (size 2 0.9) (layers F.Cu F.Paste F.Mask) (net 16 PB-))
  (pad 14 smd rect (at -8.5 8.255) (size 2 0.9) (layers F.Cu F.Paste F.Mask) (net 18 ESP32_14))
  (pad 13 smd rect (at -8.5 6.985) (size 2 0.9) (layers F.Cu F.Paste F.Mask) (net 19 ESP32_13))
  (pad 12 smd rect (at -8.5 5.715) (size 2 0.9) (layers F.Cu F.Paste F.Mask) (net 20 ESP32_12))
  (pad 11 smd rect (at -8.5 4.445) (size 2 0.9) (layers F.Cu F.Paste F.Mask) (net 21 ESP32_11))
  (pad 10 smd rect (at -8.5 3.175) (size 2 0.9) (layers F.Cu F.Paste F.Mask) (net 22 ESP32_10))
  (pad 9 smd rect (at -8.5 1.905) (size 2 0.9) (layers F.Cu F.Paste F.Mask) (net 23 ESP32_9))
  (pad 8 smd rect (at -8.5 0.635) (size 2 0.9) (layers F.Cu F.Paste F.Mask) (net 24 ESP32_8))
  (pad 7 smd rect (at -8.5 -0.635) (size 2 0.9) (layers F.Cu F.Paste F.Mask) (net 25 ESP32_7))
  (pad 6 smd rect (at -8.5 -1.905) (size 2 0.9) (layers F.Cu F.Paste F.Mask) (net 26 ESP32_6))
  (pad 5 smd rect (at -8.5 -3.175) (size 2 0.9) (layers F.Cu F.Paste F.Mask) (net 27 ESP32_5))
  (pad 4 smd rect (at -8.5 -4.445) (size 2 0.9) (layers F.Cu F.Paste F.Mask) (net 28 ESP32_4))
  (pad 3 smd rect (at -8.5 -5.715) (size 2 0.9) (layers F.Cu F.Paste F.Mask) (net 29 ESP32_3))
  (pad 2 smd rect (at -8.5 -6.985) (size 2 0.9) (layers F.Cu F.Paste F.Mask) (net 30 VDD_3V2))
  (pad 1 smd rect (at -8.5 -8.255) (size 2 0.9) (layers F.Cu F.Paste F.Mask) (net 16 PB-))
  (pad 39 smd rect (at -1 -0.755) (size 5 5) (layers F.Cu F.Paste F.Mask)))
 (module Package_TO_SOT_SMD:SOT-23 (layer F.Cu) (at 53.4416 48.0187)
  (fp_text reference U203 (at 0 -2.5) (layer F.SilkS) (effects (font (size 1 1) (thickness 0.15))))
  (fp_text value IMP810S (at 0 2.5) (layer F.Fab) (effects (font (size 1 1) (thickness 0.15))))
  (pad 3 smd rect (at 1 0) (size 0.9 0.8) (layers F.Cu F.Paste F.Mask) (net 47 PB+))
  (pad 2 smd rect (at -1 0.95) (size 0.9 0.8) (layers F.Cu F.Paste F.Mask) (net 49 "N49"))
  (pad 1 smd rect (at -1 -0.95) (size 0.9 0.8) (layers F.Cu F.Paste F.Mask) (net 16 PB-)))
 (gr_line (start 100 50) (end 100 140) (layer Edge.Cuts) (width 0.12))
 (gr_line (start 100 140) (end 150 140) (layer Edge.Cuts) (width 0.12))
 (gr_line (start 150 50) (end 150 140) (layer Edge.Cuts) (width 0.12))
 (gr_line (start 100 50) (end 150 50) (layer Edge.Cuts) (width 0.12))
 (segment (start 122.3897 136.8931) (end 122.9487 137.4521) (width 0.25) (layer F.Cu) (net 42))
 (segment (start 122.3897 134.62254) (end 122.3897 136.8931) (width 0.25) (layer F.Cu) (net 42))
 (segment (start 122.3897 133.1089) (end 122.41276 133.08584) (width 0.25) (layer F.Cu) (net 42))
 (segment (start 122.3897 134.62254) (end 122.3897 133.1089) (width 0.25) (layer F.Cu) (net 42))
 (segment (start 122.62866 132.86994) (end 122.41276 133.08584) (width 0.25) (layer F.Cu) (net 42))
 (segment (start 124.59708 132.86994) (end 122.62866 132.86994) (width 0.25) (layer F.Cu) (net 42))
 (segment (start 122.36958 133.12902) (end 122.41276 133.08584) (width 0.25) (layer F.Cu) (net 42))
 (segment (start 120.5865 133.12902) (end 122.36958 133.12902) (width 0.25) (layer F.Cu) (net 42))
 (segment (start 126.49708 134.0102) (end 127.10942 134.62254) (width 0.25) (layer F.Cu) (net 41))
 (segment (start 126.49708 132.86994) (end 126.49708 134.0102) (width 0.25) (layer F.Cu) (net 41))
 (segment (start 128.66116 134.62254) (end 128.69672 134.6581) (width 0.25) (layer F.Cu) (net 41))
 (segment (start 127.10942 134.62254) (end 128.66116 134.62254) (width 0.25) (layer F.Cu) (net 41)))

